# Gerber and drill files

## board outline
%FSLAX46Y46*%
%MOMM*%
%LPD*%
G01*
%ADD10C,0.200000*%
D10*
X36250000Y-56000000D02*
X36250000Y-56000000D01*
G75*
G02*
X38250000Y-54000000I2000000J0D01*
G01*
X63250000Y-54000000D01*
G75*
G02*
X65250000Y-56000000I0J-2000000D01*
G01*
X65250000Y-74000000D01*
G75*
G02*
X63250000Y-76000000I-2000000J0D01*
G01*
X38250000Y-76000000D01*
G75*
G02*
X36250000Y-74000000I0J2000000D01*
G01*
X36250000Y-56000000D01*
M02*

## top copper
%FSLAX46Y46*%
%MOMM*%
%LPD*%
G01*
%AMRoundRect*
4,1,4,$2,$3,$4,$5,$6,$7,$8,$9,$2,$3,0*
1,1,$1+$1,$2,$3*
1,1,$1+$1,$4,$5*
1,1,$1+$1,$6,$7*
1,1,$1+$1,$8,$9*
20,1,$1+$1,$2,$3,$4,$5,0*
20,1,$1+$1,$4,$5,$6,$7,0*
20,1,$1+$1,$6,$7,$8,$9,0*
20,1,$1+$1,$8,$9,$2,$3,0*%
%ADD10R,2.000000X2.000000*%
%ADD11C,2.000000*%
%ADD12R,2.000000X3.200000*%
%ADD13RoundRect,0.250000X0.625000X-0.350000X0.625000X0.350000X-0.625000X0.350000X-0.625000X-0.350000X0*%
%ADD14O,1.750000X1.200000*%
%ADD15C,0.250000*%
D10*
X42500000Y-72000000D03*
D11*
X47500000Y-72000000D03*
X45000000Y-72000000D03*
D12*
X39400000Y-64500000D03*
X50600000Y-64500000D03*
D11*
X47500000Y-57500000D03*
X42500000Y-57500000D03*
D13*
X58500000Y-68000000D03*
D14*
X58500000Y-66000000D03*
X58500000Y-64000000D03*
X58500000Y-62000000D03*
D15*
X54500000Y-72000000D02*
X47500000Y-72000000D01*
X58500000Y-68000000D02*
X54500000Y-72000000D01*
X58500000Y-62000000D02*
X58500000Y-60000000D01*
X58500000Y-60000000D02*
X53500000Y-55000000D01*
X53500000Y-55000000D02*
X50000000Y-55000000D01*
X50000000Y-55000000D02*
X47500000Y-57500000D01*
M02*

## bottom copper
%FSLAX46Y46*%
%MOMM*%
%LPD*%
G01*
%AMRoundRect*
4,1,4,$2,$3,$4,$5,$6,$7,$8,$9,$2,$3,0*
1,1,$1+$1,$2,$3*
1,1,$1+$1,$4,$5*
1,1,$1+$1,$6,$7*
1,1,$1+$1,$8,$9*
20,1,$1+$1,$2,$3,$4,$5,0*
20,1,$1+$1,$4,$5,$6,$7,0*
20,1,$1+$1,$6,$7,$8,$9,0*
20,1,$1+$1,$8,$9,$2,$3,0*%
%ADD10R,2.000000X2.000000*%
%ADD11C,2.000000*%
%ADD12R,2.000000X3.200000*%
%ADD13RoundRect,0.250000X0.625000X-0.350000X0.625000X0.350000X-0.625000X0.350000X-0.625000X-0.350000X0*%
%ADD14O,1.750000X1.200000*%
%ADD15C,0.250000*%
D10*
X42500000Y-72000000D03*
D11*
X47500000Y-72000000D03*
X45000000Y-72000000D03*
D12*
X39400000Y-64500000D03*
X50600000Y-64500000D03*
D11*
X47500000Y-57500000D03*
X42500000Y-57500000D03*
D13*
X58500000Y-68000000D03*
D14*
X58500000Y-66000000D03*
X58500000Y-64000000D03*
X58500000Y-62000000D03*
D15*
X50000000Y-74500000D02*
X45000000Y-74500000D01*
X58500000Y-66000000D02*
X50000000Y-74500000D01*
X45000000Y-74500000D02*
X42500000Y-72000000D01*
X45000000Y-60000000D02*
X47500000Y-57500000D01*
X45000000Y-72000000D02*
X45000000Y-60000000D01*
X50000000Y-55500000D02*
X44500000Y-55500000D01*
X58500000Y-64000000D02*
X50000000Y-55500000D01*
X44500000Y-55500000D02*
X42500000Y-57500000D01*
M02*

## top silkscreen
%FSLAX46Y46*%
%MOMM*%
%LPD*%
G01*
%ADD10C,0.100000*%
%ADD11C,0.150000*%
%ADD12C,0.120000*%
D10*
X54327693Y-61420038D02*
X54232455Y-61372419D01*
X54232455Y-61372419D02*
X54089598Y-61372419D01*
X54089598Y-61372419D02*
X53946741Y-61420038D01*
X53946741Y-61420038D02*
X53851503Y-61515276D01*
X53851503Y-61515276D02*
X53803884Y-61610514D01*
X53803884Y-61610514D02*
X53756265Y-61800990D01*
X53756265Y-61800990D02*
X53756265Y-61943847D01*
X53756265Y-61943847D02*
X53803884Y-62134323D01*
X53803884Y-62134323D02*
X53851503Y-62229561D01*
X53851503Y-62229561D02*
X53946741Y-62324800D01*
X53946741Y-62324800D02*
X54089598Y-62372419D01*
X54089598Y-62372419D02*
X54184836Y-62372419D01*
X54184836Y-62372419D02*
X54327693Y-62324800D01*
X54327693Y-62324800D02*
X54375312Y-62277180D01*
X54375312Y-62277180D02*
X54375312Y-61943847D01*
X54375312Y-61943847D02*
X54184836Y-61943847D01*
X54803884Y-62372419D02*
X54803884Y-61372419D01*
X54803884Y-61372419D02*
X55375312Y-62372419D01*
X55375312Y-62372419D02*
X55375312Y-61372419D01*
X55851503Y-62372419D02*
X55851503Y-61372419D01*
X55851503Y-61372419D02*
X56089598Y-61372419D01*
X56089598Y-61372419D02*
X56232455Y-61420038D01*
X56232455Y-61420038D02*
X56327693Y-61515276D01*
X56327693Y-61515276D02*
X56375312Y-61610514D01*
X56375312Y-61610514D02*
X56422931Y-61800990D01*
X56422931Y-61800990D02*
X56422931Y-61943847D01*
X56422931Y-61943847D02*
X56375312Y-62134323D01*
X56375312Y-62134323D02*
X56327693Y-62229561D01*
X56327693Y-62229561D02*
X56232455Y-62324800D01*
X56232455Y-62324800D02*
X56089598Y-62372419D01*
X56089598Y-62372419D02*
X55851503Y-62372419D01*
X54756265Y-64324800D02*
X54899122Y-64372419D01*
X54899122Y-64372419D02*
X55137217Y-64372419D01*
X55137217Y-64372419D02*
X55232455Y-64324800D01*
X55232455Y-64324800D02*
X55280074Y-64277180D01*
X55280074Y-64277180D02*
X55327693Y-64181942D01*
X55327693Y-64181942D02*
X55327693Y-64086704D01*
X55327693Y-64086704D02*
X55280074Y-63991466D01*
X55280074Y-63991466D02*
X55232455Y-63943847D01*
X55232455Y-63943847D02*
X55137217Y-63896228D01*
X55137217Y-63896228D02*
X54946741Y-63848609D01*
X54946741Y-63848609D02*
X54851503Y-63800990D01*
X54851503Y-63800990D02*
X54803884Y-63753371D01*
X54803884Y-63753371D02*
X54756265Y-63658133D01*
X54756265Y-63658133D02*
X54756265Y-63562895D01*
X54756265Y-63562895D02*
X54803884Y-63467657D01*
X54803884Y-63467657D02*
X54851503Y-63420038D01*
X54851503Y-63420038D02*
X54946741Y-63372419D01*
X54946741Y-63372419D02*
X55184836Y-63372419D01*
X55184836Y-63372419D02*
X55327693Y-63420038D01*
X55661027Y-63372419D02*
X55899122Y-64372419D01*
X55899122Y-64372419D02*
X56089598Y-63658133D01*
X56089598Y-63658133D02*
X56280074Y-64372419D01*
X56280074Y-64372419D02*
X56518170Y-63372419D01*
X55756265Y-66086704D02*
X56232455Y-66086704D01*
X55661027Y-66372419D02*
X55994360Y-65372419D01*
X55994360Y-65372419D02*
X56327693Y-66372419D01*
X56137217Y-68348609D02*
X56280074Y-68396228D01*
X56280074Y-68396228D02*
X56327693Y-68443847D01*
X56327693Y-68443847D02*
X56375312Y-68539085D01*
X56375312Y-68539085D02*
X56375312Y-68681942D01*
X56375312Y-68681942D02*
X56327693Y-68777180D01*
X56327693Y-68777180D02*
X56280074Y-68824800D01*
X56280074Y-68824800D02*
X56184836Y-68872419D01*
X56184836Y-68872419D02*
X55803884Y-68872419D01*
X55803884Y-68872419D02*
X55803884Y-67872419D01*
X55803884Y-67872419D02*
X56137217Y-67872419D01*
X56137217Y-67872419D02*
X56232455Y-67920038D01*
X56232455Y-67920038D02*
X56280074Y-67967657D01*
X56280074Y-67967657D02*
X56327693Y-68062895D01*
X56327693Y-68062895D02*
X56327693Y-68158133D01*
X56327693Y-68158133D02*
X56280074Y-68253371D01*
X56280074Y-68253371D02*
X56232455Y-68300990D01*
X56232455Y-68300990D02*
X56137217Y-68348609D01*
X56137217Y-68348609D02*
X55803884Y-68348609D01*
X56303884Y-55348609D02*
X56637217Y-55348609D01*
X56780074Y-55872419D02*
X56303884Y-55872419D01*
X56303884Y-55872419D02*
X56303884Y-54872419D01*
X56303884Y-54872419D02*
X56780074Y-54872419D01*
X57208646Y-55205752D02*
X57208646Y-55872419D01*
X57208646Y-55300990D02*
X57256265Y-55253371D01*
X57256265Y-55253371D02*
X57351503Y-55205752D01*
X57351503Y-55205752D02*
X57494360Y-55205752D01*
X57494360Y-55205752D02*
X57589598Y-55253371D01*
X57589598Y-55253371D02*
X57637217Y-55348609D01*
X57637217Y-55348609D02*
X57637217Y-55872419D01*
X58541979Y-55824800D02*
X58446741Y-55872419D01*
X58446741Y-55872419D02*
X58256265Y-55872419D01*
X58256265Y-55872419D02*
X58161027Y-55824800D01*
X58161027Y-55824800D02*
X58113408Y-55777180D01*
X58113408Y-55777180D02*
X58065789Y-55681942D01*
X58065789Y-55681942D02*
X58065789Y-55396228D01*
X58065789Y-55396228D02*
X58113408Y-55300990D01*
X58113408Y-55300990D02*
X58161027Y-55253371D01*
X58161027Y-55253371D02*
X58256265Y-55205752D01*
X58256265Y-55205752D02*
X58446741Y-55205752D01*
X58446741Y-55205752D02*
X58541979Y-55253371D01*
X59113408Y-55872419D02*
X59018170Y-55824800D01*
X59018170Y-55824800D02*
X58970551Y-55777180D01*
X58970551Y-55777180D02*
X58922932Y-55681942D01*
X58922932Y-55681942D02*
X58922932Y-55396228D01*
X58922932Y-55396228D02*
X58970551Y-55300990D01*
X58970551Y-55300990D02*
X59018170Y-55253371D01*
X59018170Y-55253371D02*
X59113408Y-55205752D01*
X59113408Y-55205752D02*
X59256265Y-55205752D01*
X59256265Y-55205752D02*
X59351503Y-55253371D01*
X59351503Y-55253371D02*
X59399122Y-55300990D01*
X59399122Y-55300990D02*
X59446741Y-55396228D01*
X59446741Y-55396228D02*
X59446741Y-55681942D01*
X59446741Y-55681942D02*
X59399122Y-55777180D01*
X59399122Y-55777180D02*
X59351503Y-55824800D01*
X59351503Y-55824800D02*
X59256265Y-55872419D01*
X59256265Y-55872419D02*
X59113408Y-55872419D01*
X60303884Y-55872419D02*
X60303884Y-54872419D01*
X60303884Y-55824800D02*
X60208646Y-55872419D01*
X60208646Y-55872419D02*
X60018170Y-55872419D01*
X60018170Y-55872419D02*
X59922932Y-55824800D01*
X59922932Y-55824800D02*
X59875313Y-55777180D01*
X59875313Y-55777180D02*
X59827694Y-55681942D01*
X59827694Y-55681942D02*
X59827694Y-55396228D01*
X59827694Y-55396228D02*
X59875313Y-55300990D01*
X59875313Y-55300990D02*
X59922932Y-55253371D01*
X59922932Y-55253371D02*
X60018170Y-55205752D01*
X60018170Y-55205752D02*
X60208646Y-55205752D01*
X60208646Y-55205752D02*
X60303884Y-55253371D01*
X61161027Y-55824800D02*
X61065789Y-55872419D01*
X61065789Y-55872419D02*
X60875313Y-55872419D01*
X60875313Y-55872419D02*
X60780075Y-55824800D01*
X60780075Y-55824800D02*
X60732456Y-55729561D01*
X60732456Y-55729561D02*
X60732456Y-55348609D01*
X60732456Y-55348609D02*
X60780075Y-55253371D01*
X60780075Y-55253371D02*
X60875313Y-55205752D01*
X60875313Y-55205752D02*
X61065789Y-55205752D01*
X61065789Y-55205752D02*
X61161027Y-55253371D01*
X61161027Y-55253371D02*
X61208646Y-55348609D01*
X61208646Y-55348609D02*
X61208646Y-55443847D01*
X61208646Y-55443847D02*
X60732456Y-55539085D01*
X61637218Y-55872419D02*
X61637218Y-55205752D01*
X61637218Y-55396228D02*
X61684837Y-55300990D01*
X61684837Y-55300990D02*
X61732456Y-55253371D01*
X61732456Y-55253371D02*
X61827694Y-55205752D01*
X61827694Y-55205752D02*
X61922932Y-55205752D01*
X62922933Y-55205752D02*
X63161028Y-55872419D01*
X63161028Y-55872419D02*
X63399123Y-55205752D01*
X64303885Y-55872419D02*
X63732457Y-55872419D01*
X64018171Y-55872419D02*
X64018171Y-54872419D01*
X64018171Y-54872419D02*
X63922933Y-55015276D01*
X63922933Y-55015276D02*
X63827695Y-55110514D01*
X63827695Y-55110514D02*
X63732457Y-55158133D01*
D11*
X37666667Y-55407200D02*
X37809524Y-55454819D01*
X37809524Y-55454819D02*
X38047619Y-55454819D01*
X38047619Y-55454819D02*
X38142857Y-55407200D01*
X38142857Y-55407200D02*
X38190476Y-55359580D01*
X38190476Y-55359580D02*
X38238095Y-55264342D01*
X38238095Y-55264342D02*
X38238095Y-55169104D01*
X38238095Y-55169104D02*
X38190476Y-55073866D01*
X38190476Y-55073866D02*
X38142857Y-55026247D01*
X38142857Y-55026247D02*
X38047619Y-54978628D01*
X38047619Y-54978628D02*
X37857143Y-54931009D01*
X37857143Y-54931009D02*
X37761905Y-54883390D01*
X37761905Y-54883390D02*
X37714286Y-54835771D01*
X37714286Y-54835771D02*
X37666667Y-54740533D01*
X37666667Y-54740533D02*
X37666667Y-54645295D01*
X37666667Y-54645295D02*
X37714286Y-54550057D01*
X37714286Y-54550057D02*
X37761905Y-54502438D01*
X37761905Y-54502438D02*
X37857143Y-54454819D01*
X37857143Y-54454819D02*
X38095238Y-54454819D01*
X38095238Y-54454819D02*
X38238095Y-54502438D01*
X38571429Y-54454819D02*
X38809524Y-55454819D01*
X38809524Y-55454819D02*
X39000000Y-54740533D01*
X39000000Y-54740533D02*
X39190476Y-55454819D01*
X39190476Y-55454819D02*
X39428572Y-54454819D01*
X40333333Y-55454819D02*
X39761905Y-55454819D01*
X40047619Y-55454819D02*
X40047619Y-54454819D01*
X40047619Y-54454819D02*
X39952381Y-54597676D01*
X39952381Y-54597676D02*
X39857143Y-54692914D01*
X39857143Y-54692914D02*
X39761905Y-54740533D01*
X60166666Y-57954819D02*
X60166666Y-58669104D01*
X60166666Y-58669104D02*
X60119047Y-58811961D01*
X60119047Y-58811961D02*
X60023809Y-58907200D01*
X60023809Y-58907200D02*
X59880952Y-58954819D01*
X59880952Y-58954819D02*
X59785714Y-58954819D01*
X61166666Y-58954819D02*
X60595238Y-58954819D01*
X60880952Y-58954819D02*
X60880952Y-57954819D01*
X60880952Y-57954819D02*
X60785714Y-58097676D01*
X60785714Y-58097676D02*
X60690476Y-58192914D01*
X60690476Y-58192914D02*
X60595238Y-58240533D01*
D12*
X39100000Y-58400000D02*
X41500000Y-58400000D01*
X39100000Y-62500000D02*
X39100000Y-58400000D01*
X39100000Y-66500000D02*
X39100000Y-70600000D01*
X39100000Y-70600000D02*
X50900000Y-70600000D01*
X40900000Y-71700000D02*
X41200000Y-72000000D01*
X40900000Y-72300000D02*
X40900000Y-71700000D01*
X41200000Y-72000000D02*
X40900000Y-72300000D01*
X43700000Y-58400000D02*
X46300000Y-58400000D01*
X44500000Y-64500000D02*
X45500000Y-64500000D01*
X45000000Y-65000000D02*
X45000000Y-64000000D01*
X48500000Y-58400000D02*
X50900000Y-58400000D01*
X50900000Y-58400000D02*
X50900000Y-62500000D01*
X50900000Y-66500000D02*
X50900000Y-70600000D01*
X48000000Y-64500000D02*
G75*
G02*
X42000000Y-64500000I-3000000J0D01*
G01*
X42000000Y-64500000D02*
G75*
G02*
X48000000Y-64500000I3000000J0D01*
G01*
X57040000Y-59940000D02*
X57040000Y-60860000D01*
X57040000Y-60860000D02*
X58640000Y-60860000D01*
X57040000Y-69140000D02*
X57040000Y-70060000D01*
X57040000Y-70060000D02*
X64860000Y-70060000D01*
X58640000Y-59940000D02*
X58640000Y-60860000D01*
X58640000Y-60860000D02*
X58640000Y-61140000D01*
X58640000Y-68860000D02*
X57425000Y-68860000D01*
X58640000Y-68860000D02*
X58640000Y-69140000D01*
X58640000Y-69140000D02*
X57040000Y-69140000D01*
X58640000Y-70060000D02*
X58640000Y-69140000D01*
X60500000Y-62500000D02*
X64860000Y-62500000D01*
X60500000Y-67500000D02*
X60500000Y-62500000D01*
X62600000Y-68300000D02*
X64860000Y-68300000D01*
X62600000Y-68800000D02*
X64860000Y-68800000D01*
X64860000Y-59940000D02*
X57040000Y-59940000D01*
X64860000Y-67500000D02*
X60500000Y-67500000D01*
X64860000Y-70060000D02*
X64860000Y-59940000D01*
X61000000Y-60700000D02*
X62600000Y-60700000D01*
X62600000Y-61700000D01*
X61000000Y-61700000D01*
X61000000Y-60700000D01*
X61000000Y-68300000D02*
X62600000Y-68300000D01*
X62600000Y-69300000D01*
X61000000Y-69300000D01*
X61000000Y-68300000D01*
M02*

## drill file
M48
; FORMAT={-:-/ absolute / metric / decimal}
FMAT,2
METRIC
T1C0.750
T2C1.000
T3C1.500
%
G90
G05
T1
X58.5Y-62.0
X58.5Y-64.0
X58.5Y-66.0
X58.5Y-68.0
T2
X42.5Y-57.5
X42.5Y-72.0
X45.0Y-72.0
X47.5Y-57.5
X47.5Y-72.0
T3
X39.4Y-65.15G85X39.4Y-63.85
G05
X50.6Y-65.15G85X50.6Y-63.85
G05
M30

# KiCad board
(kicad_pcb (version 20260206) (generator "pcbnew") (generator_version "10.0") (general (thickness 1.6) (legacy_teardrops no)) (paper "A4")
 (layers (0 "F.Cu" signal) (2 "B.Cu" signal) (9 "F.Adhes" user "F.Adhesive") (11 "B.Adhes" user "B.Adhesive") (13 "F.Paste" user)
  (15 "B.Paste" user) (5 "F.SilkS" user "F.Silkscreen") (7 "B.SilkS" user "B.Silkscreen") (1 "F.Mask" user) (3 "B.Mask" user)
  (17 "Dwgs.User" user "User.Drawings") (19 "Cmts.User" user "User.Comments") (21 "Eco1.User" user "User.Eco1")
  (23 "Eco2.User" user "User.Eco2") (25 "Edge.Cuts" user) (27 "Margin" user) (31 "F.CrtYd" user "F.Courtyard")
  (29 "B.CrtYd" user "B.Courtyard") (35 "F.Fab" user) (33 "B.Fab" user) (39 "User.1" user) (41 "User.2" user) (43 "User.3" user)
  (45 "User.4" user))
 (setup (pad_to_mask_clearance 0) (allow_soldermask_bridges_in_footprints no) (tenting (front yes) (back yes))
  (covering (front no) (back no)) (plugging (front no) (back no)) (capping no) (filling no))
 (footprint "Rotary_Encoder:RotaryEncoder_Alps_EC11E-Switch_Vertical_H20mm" (layer "F.Cu") (at 42.5 72 90)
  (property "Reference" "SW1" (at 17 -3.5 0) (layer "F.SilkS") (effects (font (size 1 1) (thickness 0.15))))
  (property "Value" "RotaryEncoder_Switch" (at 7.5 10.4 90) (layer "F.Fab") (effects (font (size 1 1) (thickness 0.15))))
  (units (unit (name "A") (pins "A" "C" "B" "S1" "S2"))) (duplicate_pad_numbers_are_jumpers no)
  (fp_line (start 13.6 -3.4) (end 13.6 -1) (stroke (width 0.12) (type solid)) (layer "F.SilkS"))
  (fp_line (start 9.5 -3.4) (end 13.6 -3.4) (stroke (width 0.12) (type solid)) (layer "F.SilkS"))
  (fp_line (start 5.5 -3.4) (end 1.4 -3.4) (stroke (width 0.12) (type solid)) (layer "F.SilkS"))
  (fp_line (start 1.4 -3.4) (end 1.4 8.4) (stroke (width 0.12) (type solid)) (layer "F.SilkS"))
  (fp_line (start 0.3 -1.6) (end 0 -1.3) (stroke (width 0.12) (type solid)) (layer "F.SilkS"))
  (fp_line (start -0.3 -1.6) (end 0.3 -1.6) (stroke (width 0.12) (type solid)) (layer "F.SilkS"))
  (fp_line (start 0 -1.3) (end -0.3 -1.6) (stroke (width 0.12) (type solid)) (layer "F.SilkS"))
  (fp_line (start 13.6 1.2) (end 13.6 3.8) (stroke (width 0.12) (type solid)) (layer "F.SilkS"))
  (fp_line (start 7.5 2) (end 7.5 3) (stroke (width 0.12) (type solid)) (layer "F.SilkS"))
  (fp_line (start 7 2.5) (end 8 2.5) (stroke (width 0.12) (type solid)) (layer "F.SilkS"))
  (fp_line (start 13.6 6) (end 13.6 8.4) (stroke (width 0.12) (type solid)) (layer "F.SilkS"))
  (fp_line (start 13.6 8.4) (end 9.5 8.4) (stroke (width 0.12) (type solid)) (layer "F.SilkS"))
  (fp_line (start 5.5 8.4) (end 1.4 8.4) (stroke (width 0.12) (type solid)) (layer "F.SilkS"))
  (fp_circle (center 7.5 2.5) (end 10.5 2.5) (stroke (width 0.12) (type solid)) (fill no) (layer "F.SilkS"))
  (pad "A" thru_hole rect (at 0 0 90) (size 2 2) (drill 1) (layers "*.Cu" "*.Mask") (remove_unused_layers no) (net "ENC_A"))
  (pad "B" thru_hole circle (at 0 5 90) (size 2 2) (drill 1) (layers "*.Cu" "*.Mask") (remove_unused_layers no) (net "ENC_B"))
  (pad "C" thru_hole circle (at 0 2.5 90) (size 2 2) (drill 1) (layers "*.Cu" "*.Mask") (remove_unused_layers no) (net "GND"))
  (pad "MP" thru_hole rect (at 7.5 -3.1 90) (size 3.2 2) (drill oval 2.8 1.5) (layers "*.Cu" "*.Mask") (remove_unused_layers no))
  (pad "MP" thru_hole rect (at 7.5 8.1 90) (size 3.2 2) (drill oval 2.8 1.5) (layers "*.Cu" "*.Mask") (remove_unused_layers no))
  (pad "S1" thru_hole circle (at 14.5 5 90) (size 2 2) (drill 1) (layers "*.Cu" "*.Mask") (remove_unused_layers no) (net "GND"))
  (pad "S2" thru_hole circle (at 14.5 0 90) (size 2 2) (drill 1) (layers "*.Cu" "*.Mask") (remove_unused_layers no) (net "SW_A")))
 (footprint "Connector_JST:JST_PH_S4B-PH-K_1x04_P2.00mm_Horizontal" (layer "F.Cu") (at 58.5 68 90)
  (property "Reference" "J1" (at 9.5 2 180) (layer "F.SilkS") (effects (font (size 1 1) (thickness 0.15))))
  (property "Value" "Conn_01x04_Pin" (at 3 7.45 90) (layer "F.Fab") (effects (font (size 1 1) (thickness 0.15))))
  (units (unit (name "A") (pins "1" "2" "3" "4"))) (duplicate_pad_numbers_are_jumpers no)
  (fp_line (start 8.06 -1.46) (end 7.14 -1.46) (stroke (width 0.12) (type solid)) (layer "F.SilkS"))
  (fp_line (start 7.14 -1.46) (end 7.14 0.14) (stroke (width 0.12) (type solid)) (layer "F.SilkS"))
  (fp_line (start -1.14 -1.46) (end -2.06 -1.46) (stroke (width 0.12) (type solid)) (layer "F.SilkS"))
  (fp_line (start -2.06 -1.46) (end -2.06 6.36) (stroke (width 0.12) (type solid)) (layer "F.SilkS"))
  (fp_line (start 8.06 0.14) (end 7.14 0.14) (stroke (width 0.12) (type solid)) (layer "F.SilkS"))
  (fp_line (start 7.14 0.14) (end 6.86 0.14) (stroke (width 0.12) (type solid)) (layer "F.SilkS"))
  (fp_line (start -0.86 0.14) (end -0.86 -1.075) (stroke (width 0.12) (type solid)) (layer "F.SilkS"))
  (fp_line (start -0.86 0.14) (end -1.14 0.14) (stroke (width 0.12) (type solid)) (layer "F.SilkS"))
  (fp_line (start -1.14 0.14) (end -1.14 -1.46) (stroke (width 0.12) (type solid)) (layer "F.SilkS"))
  (fp_line (start -2.06 0.14) (end -1.14 0.14) (stroke (width 0.12) (type solid)) (layer "F.SilkS"))
  (fp_line (start 5.5 2) (end 5.5 6.36) (stroke (width 0.12) (type solid)) (layer "F.SilkS"))
  (fp_line (start 0.5 2) (end 5.5 2) (stroke (width 0.12) (type solid)) (layer "F.SilkS"))
  (fp_line (start -0.3 4.1) (end -0.3 6.36) (stroke (width 0.12) (type solid)) (layer "F.SilkS"))
  (fp_line (start -0.8 4.1) (end -0.8 6.36) (stroke (width 0.12) (type solid)) (layer "F.SilkS"))
  (fp_line (start 8.06 6.36) (end 8.06 -1.46) (stroke (width 0.12) (type solid)) (layer "F.SilkS"))
  (fp_line (start 0.5 6.36) (end 0.5 2) (stroke (width 0.12) (type solid)) (layer "F.SilkS"))
  (fp_line (start -2.06 6.36) (end 8.06 6.36) (stroke (width 0.12) (type solid)) (layer "F.SilkS"))
  (fp_rect (start 6.3 2.5) (end 7.3 4.1) (stroke (width 0.12) (type solid)) (fill no) (layer "F.SilkS"))
  (fp_rect (start -1.3 2.5) (end -0.3 4.1) (stroke (width 0.12) (type solid)) (fill no) (layer "F.SilkS"))
  (pad "1" thru_hole roundrect (at 0 0 90) (size 1.2 1.75) (drill 0.75) (layers "*.Cu" "*.Mask") (remove_unused_layers no)
   (roundrect_rratio 0.208333) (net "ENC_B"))
  (pad "2" thru_hole oval (at 2 0 90) (size 1.2 1.75) (drill 0.75) (layers "*.Cu" "*.Mask") (remove_unused_layers no) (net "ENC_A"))
  (pad "3" thru_hole oval (at 4 0 90) (size 1.2 1.75) (drill 0.75) (layers "*.Cu" "*.Mask") (remove_unused_layers no) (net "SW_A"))
  (pad "4" thru_hole oval (at 6 0 90) (size 1.2 1.75) (drill 0.75) (layers "*.Cu" "*.Mask") (remove_unused_layers no) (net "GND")))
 (gr_rect (start 36.25 54) (end 65.25 76) (radius 2) (stroke (width 0.2) (type solid)) (fill no) (layer "Edge.Cuts"))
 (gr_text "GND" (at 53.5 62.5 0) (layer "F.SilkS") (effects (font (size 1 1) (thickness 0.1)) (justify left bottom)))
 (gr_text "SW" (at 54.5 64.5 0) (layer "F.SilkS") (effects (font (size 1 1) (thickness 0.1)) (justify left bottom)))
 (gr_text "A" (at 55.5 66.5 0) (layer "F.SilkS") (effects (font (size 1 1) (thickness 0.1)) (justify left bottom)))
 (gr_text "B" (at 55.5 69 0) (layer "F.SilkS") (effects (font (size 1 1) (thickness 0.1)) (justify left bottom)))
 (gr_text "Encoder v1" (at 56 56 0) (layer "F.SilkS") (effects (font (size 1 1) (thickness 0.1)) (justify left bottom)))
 (segment (start 50 74.5) (end 45 74.5) (width 0.25) (layer "B.Cu") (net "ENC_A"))
 (segment (start 58.5 66) (end 50 74.5) (width 0.25) (layer "B.Cu") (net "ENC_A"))
 (segment (start 45 74.5) (end 42.5 72) (width 0.25) (layer "B.Cu") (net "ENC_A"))
 (segment (start 54.5 72) (end 47.5 72) (width 0.25) (layer "F.Cu") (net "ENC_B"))
 (segment (start 58.5 68) (end 54.5 72) (width 0.25) (layer "F.Cu") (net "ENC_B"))
 (segment (start 58.5 62) (end 58.5 60) (width 0.25) (layer "F.Cu") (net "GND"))
 (segment (start 58.5 60) (end 53.5 55) (width 0.25) (layer "F.Cu") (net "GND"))
 (segment (start 53.5 55) (end 50 55) (width 0.25) (layer "F.Cu") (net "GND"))
 (segment (start 50 55) (end 47.5 57.5) (width 0.25) (layer "F.Cu") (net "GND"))
 (segment (start 45 60) (end 47.5 57.5) (width 0.25) (layer "B.Cu") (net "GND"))
 (segment (start 45 72) (end 45 60) (width 0.25) (layer "B.Cu") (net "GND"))
 (segment (start 50 55.5) (end 44.5 55.5) (width 0.25) (layer "B.Cu") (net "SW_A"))
 (segment (start 58.5 64) (end 50 55.5) (width 0.25) (layer "B.Cu") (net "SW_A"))
 (segment (start 44.5 55.5) (end 42.5 57.5) (width 0.25) (layer "B.Cu") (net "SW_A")))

